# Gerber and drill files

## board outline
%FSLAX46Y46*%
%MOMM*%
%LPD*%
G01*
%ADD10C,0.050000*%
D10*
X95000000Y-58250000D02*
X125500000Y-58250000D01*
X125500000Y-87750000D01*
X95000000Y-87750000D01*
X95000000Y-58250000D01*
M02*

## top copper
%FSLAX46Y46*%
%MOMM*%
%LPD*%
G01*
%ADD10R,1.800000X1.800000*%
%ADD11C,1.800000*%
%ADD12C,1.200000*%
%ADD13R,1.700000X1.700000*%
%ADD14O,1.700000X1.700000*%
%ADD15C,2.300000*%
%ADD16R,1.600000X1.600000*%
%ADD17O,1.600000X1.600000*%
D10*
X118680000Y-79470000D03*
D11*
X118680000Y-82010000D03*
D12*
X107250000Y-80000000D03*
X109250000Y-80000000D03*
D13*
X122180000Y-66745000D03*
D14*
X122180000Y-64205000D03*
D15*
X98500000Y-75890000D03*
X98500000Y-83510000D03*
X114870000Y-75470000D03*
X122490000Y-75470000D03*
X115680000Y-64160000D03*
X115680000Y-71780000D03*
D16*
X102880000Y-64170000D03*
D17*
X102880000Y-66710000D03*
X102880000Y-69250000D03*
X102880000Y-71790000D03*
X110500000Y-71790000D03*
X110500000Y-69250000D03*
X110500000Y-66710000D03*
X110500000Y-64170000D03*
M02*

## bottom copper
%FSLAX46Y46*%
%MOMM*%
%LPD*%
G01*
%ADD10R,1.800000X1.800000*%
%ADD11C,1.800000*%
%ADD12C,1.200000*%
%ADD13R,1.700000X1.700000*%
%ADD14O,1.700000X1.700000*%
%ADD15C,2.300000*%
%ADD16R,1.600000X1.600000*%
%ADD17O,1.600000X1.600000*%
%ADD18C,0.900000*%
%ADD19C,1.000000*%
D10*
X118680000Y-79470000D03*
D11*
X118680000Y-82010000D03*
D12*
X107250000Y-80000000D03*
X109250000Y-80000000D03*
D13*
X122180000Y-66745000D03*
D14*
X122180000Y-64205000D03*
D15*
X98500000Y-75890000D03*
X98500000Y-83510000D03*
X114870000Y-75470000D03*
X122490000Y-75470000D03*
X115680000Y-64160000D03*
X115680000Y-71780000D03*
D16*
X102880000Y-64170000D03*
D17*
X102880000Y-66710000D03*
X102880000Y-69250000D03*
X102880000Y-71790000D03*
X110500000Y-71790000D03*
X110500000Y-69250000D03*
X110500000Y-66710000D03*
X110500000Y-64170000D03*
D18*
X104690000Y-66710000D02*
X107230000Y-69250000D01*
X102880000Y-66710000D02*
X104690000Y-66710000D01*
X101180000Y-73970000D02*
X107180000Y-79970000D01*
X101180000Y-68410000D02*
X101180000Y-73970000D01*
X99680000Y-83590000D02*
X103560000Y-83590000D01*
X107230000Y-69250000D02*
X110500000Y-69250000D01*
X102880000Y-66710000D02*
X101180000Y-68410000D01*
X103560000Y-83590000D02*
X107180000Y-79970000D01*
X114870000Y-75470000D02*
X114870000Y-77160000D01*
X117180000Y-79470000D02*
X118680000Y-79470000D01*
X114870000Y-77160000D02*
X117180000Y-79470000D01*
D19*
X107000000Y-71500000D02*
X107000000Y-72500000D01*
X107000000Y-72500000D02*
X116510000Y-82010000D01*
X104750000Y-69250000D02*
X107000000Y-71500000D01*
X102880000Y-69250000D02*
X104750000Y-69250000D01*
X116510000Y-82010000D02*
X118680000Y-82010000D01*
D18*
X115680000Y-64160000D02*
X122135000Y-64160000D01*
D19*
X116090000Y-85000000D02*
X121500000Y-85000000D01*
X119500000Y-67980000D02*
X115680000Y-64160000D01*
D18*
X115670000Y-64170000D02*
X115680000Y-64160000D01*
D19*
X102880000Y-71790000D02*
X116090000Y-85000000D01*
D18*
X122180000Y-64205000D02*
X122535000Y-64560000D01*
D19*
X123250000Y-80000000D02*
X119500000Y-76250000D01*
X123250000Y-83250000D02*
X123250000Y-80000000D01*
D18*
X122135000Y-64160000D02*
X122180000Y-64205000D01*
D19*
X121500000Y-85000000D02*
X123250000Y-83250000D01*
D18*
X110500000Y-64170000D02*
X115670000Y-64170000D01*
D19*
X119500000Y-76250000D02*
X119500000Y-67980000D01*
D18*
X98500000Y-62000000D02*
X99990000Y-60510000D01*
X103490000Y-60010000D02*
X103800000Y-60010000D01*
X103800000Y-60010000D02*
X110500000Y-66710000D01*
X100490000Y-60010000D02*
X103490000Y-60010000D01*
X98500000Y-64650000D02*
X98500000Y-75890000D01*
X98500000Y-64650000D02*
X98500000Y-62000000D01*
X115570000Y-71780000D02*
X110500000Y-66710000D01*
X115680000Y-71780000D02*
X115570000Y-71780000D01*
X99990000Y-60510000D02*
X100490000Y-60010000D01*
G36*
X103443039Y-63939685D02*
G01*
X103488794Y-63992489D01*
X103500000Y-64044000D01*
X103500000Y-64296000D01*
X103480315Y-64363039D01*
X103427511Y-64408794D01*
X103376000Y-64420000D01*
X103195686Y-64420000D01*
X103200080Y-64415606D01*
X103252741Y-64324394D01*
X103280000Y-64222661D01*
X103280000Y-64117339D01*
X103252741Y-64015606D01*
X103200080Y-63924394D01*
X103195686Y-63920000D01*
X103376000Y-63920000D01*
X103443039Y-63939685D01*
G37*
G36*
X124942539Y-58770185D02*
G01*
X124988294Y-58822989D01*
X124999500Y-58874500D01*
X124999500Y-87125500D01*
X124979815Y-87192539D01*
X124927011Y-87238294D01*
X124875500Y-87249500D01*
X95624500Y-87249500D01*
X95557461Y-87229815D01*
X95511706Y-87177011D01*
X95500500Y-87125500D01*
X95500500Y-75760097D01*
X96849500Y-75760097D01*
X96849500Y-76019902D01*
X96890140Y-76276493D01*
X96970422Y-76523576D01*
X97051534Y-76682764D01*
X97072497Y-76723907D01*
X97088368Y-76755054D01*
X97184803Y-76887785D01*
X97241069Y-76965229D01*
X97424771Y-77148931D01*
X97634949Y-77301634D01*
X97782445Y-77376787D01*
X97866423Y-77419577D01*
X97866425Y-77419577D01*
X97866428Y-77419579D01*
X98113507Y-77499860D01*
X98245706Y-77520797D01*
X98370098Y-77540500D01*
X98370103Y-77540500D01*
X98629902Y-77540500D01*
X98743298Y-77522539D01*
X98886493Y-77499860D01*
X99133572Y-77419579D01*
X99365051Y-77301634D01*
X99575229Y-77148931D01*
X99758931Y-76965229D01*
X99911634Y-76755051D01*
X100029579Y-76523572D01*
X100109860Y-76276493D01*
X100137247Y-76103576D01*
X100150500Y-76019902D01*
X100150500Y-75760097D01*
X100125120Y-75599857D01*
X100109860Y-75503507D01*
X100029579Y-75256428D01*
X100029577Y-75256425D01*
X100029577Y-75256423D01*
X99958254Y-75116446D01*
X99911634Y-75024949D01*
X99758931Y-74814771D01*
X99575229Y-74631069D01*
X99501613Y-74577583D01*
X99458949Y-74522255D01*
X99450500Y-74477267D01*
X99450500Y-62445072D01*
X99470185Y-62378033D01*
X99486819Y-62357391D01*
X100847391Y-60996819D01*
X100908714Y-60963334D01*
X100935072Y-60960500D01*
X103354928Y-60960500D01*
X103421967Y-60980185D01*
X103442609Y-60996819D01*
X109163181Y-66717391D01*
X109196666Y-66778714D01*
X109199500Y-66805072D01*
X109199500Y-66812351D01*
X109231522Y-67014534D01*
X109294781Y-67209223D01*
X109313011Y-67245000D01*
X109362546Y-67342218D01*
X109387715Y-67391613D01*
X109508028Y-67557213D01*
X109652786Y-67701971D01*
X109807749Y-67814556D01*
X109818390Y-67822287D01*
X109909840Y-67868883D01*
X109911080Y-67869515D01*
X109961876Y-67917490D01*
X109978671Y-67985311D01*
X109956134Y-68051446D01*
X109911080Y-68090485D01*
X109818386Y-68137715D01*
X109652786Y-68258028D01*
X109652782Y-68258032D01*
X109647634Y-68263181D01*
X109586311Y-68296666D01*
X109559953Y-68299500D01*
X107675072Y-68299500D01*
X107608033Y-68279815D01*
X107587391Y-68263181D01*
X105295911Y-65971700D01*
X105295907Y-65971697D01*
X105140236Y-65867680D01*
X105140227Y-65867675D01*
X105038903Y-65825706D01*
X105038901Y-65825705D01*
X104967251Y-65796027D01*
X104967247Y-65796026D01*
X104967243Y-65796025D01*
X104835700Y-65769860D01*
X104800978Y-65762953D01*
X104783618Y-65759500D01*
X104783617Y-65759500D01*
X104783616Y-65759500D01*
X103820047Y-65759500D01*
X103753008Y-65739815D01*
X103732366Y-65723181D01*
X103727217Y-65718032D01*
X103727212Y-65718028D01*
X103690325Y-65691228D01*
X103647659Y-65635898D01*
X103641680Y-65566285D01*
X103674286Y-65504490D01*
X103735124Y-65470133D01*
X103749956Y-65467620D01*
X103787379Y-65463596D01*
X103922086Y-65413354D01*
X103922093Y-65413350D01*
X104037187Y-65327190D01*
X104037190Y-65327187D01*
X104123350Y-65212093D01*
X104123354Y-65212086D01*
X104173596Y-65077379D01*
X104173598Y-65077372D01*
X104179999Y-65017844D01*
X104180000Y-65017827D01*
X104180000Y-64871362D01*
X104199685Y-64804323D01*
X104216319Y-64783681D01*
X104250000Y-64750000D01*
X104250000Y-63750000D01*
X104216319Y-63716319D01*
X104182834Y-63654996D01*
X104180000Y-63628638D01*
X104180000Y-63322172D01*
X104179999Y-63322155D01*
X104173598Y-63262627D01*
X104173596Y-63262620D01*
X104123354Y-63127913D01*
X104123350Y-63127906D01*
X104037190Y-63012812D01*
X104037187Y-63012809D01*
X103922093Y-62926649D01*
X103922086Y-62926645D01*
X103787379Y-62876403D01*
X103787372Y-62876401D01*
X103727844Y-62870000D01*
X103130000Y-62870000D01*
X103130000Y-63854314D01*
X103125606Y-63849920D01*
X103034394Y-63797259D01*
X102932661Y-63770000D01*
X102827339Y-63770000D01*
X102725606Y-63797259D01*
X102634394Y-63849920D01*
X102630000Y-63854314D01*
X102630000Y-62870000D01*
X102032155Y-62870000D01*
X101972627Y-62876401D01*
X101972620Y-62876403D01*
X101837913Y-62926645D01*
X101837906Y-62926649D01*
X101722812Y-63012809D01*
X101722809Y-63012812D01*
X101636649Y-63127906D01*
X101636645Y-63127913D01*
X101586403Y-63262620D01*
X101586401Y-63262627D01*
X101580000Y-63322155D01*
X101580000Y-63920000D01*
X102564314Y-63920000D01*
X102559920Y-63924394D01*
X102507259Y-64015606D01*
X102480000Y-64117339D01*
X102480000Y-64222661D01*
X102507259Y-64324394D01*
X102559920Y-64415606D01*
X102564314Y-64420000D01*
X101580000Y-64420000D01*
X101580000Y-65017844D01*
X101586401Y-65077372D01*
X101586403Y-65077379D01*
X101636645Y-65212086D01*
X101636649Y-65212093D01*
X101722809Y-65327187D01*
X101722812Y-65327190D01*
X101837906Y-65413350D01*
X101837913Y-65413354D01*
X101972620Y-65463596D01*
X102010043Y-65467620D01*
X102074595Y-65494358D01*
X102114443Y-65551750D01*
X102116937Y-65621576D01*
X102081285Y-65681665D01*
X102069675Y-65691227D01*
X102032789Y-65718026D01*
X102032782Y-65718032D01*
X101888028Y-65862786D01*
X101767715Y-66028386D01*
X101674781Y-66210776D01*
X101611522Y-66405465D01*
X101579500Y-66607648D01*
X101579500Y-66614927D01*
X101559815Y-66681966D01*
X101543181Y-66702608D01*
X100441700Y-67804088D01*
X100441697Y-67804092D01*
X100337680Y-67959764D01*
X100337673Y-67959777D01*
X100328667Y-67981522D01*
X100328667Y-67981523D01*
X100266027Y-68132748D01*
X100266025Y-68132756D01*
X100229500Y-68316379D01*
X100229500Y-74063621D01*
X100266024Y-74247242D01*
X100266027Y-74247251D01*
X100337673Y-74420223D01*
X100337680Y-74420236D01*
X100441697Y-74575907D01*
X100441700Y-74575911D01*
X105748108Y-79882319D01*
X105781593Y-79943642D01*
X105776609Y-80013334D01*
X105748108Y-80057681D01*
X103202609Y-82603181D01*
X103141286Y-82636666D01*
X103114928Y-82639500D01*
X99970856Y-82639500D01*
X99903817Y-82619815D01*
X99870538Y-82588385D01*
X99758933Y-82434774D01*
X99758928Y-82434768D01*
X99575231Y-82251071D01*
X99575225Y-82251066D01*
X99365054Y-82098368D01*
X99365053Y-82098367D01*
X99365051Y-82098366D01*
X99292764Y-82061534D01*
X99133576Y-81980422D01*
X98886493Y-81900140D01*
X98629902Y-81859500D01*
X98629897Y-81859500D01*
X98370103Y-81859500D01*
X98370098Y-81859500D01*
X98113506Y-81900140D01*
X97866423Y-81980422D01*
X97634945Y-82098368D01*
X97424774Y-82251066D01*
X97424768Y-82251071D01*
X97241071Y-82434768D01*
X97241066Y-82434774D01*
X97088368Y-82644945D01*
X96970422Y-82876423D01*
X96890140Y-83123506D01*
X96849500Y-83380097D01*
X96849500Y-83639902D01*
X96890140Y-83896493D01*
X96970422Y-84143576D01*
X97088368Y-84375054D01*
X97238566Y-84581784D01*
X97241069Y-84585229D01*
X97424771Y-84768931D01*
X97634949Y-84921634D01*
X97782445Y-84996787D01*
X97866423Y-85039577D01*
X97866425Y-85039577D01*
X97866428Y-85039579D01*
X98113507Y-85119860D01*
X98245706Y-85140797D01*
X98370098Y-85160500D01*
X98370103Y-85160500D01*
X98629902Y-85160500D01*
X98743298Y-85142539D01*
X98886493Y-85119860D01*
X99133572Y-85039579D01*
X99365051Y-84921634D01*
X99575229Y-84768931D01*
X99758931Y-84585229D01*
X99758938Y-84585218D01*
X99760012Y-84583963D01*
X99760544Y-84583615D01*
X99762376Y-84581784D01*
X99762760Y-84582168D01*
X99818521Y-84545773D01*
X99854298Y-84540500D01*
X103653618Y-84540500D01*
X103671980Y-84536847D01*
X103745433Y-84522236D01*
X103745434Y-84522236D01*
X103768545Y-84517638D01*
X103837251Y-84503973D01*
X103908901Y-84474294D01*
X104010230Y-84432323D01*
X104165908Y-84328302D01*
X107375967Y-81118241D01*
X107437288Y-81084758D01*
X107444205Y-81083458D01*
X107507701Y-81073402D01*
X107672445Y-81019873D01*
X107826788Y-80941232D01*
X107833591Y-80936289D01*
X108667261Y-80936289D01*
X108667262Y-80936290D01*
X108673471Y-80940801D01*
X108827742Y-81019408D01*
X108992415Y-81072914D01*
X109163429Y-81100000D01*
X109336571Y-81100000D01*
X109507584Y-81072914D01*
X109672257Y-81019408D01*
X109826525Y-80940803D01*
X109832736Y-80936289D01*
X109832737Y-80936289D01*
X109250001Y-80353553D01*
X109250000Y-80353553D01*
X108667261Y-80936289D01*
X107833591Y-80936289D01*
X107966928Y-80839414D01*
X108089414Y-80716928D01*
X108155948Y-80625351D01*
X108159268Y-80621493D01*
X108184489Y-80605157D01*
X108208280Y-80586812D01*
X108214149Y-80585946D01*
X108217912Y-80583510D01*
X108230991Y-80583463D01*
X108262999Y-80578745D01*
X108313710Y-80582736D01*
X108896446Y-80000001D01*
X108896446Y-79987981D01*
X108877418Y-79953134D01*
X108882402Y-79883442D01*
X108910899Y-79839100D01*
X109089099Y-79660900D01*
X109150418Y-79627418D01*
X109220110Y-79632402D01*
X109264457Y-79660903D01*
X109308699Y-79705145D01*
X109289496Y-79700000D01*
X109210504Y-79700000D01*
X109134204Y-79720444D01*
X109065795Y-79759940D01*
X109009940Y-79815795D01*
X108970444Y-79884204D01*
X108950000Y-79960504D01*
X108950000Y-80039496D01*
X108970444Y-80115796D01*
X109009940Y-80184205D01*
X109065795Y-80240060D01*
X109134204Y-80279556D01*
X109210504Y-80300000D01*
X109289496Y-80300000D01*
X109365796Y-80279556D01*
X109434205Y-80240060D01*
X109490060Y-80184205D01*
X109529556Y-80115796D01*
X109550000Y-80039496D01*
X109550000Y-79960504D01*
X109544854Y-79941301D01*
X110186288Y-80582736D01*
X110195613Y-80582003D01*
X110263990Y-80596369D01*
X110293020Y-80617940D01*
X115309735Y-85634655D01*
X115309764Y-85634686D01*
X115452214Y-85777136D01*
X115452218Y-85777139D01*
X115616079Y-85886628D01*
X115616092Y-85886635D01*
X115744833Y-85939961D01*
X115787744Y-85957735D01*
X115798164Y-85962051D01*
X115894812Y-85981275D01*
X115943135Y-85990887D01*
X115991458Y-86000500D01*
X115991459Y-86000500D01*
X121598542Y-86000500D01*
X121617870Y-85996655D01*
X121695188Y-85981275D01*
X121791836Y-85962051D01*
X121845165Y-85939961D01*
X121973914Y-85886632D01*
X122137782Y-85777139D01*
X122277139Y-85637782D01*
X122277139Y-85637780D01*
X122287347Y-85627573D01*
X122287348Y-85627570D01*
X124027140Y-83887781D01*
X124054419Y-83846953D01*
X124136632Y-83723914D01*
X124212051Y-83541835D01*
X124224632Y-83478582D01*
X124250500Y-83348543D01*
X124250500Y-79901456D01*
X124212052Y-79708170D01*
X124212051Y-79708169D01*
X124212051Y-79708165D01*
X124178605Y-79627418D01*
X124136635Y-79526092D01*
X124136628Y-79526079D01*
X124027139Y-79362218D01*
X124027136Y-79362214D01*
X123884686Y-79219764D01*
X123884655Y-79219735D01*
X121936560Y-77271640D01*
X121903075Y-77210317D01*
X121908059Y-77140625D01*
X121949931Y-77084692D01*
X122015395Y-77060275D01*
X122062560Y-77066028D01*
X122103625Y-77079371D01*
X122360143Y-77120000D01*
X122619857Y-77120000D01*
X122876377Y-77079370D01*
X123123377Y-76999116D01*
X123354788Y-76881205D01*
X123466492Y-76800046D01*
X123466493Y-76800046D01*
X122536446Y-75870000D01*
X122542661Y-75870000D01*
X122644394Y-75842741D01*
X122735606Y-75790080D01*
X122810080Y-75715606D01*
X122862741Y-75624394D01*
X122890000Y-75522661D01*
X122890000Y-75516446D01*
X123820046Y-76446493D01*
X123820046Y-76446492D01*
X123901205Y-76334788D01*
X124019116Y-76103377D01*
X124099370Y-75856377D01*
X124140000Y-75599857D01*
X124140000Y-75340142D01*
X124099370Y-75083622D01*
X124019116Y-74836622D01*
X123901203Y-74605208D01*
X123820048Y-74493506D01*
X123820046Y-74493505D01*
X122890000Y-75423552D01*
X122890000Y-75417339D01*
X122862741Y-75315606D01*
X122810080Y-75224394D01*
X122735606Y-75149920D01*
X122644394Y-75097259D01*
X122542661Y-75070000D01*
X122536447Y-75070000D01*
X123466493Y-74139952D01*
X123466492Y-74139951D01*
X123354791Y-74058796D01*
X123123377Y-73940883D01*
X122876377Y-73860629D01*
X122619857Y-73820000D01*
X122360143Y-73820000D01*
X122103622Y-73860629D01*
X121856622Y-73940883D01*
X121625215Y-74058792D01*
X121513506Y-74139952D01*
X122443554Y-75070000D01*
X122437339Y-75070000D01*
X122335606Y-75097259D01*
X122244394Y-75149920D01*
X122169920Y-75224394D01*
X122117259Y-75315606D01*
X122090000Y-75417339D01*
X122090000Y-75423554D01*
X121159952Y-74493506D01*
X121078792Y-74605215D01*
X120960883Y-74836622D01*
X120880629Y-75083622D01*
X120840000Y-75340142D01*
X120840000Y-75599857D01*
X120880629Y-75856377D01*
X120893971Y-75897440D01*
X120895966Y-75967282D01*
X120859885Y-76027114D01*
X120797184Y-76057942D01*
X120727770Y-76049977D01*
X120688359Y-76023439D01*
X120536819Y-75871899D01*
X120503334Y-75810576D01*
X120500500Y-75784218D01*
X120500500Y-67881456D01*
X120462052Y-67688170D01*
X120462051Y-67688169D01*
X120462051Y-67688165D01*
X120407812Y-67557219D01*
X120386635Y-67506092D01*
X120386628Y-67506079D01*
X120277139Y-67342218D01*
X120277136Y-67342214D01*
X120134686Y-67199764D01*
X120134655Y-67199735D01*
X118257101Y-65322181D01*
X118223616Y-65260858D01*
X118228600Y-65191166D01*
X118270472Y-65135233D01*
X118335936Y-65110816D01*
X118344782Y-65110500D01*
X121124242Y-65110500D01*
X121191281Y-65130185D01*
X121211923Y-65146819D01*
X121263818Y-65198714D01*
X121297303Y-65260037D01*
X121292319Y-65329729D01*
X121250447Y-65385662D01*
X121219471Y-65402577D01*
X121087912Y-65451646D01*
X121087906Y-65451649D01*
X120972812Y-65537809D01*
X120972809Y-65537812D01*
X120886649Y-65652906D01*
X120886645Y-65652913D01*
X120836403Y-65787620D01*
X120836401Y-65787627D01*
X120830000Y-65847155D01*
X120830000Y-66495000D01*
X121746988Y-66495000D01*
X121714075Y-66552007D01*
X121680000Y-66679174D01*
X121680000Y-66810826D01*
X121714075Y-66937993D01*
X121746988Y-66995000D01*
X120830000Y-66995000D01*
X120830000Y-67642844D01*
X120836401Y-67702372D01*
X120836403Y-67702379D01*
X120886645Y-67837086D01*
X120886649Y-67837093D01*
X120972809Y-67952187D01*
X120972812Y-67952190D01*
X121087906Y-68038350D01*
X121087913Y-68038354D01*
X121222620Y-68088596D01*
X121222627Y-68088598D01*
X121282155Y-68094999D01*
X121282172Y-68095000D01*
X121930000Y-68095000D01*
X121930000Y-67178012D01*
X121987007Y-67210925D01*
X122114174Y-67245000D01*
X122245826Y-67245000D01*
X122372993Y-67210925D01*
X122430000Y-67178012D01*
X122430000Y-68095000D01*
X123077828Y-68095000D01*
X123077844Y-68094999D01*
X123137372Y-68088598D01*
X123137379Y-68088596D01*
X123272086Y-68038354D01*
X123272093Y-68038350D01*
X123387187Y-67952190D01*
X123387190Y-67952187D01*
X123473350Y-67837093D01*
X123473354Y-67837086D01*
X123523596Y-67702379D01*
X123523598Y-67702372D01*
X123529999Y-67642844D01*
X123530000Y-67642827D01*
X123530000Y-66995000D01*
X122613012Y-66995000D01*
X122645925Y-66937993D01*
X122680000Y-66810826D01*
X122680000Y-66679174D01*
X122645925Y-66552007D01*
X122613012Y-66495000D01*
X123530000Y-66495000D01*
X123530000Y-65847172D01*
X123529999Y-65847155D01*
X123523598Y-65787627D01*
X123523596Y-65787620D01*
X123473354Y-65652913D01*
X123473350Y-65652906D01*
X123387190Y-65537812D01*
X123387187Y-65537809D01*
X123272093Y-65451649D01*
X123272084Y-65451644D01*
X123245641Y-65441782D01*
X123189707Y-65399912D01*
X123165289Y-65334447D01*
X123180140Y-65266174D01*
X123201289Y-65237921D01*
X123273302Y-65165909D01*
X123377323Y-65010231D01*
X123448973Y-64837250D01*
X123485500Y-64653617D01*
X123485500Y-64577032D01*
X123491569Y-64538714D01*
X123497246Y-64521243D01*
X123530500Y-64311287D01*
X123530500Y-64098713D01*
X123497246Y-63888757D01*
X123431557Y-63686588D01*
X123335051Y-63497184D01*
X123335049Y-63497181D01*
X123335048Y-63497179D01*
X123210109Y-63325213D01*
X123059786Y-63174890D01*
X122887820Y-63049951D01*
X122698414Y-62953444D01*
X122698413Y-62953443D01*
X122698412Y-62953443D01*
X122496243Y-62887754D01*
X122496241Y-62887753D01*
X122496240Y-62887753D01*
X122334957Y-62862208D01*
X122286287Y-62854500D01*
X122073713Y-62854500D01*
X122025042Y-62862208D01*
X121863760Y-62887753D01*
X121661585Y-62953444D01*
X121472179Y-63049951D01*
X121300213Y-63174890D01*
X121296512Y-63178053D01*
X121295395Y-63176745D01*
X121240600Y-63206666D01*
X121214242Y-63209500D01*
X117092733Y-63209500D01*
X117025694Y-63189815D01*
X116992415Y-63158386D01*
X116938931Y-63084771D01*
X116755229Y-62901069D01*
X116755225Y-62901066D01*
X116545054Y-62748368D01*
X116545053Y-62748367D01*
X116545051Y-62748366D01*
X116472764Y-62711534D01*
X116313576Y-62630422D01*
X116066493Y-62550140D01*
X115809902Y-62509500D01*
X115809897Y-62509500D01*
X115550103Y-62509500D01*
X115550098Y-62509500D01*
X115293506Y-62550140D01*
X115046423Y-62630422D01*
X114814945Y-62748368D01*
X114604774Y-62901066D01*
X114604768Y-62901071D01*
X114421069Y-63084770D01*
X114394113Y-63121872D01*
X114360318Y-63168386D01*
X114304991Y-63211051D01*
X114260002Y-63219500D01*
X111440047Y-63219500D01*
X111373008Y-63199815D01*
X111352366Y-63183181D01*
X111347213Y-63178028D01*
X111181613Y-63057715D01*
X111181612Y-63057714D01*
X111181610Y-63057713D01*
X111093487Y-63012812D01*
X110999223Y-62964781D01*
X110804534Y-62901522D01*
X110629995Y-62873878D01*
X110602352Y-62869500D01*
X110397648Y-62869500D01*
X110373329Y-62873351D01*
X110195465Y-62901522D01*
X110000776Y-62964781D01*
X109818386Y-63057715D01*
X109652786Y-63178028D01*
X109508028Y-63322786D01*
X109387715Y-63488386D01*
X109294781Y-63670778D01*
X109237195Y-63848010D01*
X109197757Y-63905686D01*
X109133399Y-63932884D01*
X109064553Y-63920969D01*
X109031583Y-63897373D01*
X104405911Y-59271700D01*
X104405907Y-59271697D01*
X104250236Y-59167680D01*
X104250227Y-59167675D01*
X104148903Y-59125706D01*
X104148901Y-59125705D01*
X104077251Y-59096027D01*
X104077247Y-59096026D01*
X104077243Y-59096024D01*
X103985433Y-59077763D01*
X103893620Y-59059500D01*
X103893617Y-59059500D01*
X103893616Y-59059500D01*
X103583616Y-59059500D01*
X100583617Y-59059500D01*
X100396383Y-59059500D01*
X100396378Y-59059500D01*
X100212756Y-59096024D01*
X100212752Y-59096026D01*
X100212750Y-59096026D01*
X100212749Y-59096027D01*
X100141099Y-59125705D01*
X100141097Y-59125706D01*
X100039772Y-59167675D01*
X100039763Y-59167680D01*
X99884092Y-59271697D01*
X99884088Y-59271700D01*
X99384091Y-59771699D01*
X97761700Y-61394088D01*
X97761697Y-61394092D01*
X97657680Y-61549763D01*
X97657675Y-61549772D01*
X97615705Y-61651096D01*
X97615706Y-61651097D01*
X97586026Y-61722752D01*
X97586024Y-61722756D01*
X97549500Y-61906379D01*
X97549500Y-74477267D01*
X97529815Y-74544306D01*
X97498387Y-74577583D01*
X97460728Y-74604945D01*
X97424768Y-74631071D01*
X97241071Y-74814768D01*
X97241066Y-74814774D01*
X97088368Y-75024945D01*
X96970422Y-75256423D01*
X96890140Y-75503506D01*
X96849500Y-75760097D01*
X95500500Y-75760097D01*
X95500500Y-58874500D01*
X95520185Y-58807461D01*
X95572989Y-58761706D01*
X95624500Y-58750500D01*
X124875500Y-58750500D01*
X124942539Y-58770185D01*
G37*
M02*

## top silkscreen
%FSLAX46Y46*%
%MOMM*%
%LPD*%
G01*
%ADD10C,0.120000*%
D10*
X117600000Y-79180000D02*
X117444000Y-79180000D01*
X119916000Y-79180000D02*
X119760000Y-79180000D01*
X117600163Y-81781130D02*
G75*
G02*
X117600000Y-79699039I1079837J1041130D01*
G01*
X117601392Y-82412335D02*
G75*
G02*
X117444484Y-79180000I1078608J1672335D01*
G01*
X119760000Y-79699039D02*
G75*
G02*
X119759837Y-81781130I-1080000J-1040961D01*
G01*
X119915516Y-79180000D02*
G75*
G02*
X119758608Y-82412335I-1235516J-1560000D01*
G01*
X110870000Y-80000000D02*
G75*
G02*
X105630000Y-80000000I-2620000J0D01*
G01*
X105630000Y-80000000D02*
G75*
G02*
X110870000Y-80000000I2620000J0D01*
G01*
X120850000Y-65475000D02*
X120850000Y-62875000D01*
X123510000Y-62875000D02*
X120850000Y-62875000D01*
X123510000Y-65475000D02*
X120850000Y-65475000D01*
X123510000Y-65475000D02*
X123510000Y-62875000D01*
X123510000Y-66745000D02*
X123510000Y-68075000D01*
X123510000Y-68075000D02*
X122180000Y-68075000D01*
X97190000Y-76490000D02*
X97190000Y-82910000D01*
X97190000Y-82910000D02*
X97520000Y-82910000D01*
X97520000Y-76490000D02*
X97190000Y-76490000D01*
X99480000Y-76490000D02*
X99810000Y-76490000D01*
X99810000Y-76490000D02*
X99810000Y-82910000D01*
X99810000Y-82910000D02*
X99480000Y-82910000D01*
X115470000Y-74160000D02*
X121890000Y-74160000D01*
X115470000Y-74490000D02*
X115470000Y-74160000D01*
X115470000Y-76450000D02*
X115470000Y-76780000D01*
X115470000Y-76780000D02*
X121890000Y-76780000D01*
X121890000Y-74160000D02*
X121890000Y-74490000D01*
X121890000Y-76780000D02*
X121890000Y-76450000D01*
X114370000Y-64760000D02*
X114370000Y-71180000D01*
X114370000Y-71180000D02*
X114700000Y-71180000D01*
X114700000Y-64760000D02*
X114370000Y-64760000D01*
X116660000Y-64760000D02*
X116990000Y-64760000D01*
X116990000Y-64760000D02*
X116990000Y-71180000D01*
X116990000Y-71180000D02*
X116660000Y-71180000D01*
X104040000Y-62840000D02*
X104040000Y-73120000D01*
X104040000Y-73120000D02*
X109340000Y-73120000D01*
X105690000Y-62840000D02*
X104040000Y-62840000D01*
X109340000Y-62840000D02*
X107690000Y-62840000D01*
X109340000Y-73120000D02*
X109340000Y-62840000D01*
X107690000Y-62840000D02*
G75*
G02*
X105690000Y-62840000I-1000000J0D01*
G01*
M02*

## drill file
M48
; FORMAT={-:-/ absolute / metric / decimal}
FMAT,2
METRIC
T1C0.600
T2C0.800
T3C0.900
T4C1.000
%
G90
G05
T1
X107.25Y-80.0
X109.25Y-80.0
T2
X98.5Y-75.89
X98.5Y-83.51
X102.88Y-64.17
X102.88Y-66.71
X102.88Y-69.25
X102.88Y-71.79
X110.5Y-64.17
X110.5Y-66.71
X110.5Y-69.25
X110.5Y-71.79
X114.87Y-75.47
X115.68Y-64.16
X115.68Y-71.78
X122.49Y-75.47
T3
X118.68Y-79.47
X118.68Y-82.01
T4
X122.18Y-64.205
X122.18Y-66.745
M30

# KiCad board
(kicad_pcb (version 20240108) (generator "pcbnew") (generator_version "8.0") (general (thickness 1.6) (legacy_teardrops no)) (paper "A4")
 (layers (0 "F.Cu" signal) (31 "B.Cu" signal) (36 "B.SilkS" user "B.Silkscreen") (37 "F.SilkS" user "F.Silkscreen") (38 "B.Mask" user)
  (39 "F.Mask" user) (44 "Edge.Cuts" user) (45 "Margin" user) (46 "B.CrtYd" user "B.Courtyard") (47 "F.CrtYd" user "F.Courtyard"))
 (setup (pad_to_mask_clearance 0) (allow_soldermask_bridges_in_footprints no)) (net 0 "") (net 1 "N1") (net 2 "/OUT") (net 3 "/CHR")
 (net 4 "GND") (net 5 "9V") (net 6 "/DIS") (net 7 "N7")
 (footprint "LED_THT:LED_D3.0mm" (layer "F.Cu") (at 118.68 79.47 -90)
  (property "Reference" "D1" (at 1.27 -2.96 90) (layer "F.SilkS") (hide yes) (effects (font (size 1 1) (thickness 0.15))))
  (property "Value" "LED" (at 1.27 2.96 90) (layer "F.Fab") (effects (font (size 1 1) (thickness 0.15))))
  (fp_line (start -0.29 1.08) (end -0.29 1.236) (stroke (width 0.12) (type solid)) (layer "F.SilkS"))
  (fp_line (start -0.29 -1.236) (end -0.29 -1.08) (stroke (width 0.12) (type solid)) (layer "F.SilkS"))
  (fp_arc (start 2.31113 1.079837) (mid 1.270117 1.5) (end 0.229039 1.08) (stroke (width 0.12) (type solid)) (layer "F.SilkS"))
  (fp_arc (start 2.942335 1.078608) (mid 1.366487 1.987659) (end -0.29 1.235516) (stroke (width 0.12) (type solid)) (layer "F.SilkS"))
  (fp_arc (start 0.229039 -1.08) (mid 1.270117 -1.5) (end 2.31113 -1.079837) (stroke (width 0.12) (type solid)) (layer "F.SilkS"))
  (fp_arc (start -0.29 -1.235516) (mid 1.366487 -1.987659) (end 2.942335 -1.078608) (stroke (width 0.12) (type solid)) (layer "F.SilkS"))
  (pad "1" thru_hole rect (at 0 0 270) (size 1.8 1.8) (drill 0.9) (layers "*.Cu" "*.Mask") (remove_unused_layers no) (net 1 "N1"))
  (pad "2" thru_hole circle (at 2.54 0 270) (size 1.8 1.8) (drill 0.9) (layers "*.Cu" "*.Mask") (remove_unused_layers no) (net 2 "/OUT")))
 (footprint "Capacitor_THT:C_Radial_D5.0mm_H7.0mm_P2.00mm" (layer "F.Cu") (at 107.25 80)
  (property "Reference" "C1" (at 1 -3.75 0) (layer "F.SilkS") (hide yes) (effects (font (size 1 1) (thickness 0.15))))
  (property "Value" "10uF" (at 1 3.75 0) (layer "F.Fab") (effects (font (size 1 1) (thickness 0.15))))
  (fp_circle (center 1 0) (end 3.62 0) (stroke (width 0.12) (type solid)) (fill none) (layer "F.SilkS"))
  (pad "1" thru_hole circle (at 0 0) (size 1.2 1.2) (drill 0.6) (layers "*.Cu" "*.Mask") (remove_unused_layers no) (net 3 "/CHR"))
  (pad "2" thru_hole circle (at 2 0) (size 1.2 1.2) (drill 0.6) (layers "*.Cu" "*.Mask") (remove_unused_layers no) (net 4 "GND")))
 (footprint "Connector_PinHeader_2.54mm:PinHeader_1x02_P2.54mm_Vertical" (layer "F.Cu") (at 122.18 66.745 180)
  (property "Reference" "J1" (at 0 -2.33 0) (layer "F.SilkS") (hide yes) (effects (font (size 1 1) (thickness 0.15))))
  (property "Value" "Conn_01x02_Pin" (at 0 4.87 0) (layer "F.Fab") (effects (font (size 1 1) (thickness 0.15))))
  (fp_line (start 1.33 1.27) (end 1.33 3.87) (stroke (width 0.12) (type solid)) (layer "F.SilkS"))
  (fp_line (start -1.33 3.87) (end 1.33 3.87) (stroke (width 0.12) (type solid)) (layer "F.SilkS"))
  (fp_line (start -1.33 1.27) (end 1.33 1.27) (stroke (width 0.12) (type solid)) (layer "F.SilkS"))
  (fp_line (start -1.33 1.27) (end -1.33 3.87) (stroke (width 0.12) (type solid)) (layer "F.SilkS"))
  (fp_line (start -1.33 0) (end -1.33 -1.33) (stroke (width 0.12) (type solid)) (layer "F.SilkS"))
  (fp_line (start -1.33 -1.33) (end 0 -1.33) (stroke (width 0.12) (type solid)) (layer "F.SilkS"))
  (pad "1" thru_hole rect (at 0 0 180) (size 1.7 1.7) (drill 1) (layers "*.Cu" "*.Mask") (remove_unused_layers no) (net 4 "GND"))
  (pad "2" thru_hole oval (at 0 2.54 180) (size 1.7 1.7) (drill 1) (layers "*.Cu" "*.Mask") (remove_unused_layers no) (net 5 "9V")))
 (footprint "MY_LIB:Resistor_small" (layer "F.Cu") (at 98.5 75.89 -90)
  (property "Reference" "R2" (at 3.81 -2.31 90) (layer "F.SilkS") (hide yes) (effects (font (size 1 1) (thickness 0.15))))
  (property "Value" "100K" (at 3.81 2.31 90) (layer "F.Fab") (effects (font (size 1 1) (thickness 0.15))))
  (fp_line (start 0.6 1.31) (end 7.02 1.31) (stroke (width 0.12) (type solid)) (layer "F.SilkS"))
  (fp_line (start 7.02 1.31) (end 7.02 0.98) (stroke (width 0.12) (type solid)) (layer "F.SilkS"))
  (fp_line (start 0.6 0.98) (end 0.6 1.31) (stroke (width 0.12) (type solid)) (layer "F.SilkS"))
  (fp_line (start 0.6 -0.98) (end 0.6 -1.31) (stroke (width 0.12) (type solid)) (layer "F.SilkS"))
  (fp_line (start 0.6 -1.31) (end 7.02 -1.31) (stroke (width 0.12) (type solid)) (layer "F.SilkS"))
  (fp_line (start 7.02 -1.31) (end 7.02 -0.98) (stroke (width 0.12) (type solid)) (layer "F.SilkS"))
  (pad "1" thru_hole circle (at 0 0 270) (size 2.3 2.3) (drill 0.8) (layers "*.Cu" "*.Mask") (remove_unused_layers no) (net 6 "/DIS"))
  (pad "2" thru_hole circle (at 7.62 0 270) (size 2.3 2.3) (drill 0.8) (layers "*.Cu" "*.Mask") (remove_unused_layers no) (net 3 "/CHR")))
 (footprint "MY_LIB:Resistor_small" (layer "F.Cu") (at 114.87 75.47)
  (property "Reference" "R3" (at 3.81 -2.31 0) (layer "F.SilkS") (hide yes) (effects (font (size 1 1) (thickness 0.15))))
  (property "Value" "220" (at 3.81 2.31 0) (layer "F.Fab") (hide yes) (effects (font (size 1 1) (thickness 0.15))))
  (fp_line (start 0.6 -1.31) (end 7.02 -1.31) (stroke (width 0.12) (type solid)) (layer "F.SilkS"))
  (fp_line (start 0.6 -0.98) (end 0.6 -1.31) (stroke (width 0.12) (type solid)) (layer "F.SilkS"))
  (fp_line (start 0.6 0.98) (end 0.6 1.31) (stroke (width 0.12) (type solid)) (layer "F.SilkS"))
  (fp_line (start 0.6 1.31) (end 7.02 1.31) (stroke (width 0.12) (type solid)) (layer "F.SilkS"))
  (fp_line (start 7.02 -1.31) (end 7.02 -0.98) (stroke (width 0.12) (type solid)) (layer "F.SilkS"))
  (fp_line (start 7.02 1.31) (end 7.02 0.98) (stroke (width 0.12) (type solid)) (layer "F.SilkS"))
  (pad "1" thru_hole circle (at 0 0) (size 2.3 2.3) (drill 0.8) (layers "*.Cu" "*.Mask") (remove_unused_layers no) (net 1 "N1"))
  (pad "2" thru_hole circle (at 7.62 0) (size 2.3 2.3) (drill 0.8) (layers "*.Cu" "*.Mask") (remove_unused_layers no) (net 4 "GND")))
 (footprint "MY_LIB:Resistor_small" (layer "F.Cu") (at 115.68 64.16 -90)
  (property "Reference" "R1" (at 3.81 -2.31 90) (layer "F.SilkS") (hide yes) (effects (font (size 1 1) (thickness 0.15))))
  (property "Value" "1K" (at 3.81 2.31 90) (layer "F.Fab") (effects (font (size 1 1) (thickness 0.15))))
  (fp_line (start 0.6 1.31) (end 7.02 1.31) (stroke (width 0.12) (type solid)) (layer "F.SilkS"))
  (fp_line (start 7.02 1.31) (end 7.02 0.98) (stroke (width 0.12) (type solid)) (layer "F.SilkS"))
  (fp_line (start 0.6 0.98) (end 0.6 1.31) (stroke (width 0.12) (type solid)) (layer "F.SilkS"))
  (fp_line (start 0.6 -0.98) (end 0.6 -1.31) (stroke (width 0.12) (type solid)) (layer "F.SilkS"))
  (fp_line (start 0.6 -1.31) (end 7.02 -1.31) (stroke (width 0.12) (type solid)) (layer "F.SilkS"))
  (fp_line (start 7.02 -1.31) (end 7.02 -0.98) (stroke (width 0.12) (type solid)) (layer "F.SilkS"))
  (pad "1" thru_hole circle (at 0 0 270) (size 2.3 2.3) (drill 0.8) (layers "*.Cu" "*.Mask") (remove_unused_layers no) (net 5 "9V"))
  (pad "2" thru_hole circle (at 7.62 0 270) (size 2.3 2.3) (drill 0.8) (layers "*.Cu" "*.Mask") (remove_unused_layers no) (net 6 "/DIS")))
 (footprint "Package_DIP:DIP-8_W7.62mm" (layer "F.Cu") (at 102.88 64.17)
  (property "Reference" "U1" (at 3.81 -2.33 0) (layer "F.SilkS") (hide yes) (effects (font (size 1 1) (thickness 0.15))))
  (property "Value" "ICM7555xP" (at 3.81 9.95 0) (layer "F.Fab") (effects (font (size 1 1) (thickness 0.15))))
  (fp_line (start 1.16 -1.33) (end 1.16 8.95) (stroke (width 0.12) (type solid)) (layer "F.SilkS"))
  (fp_line (start 1.16 8.95) (end 6.46 8.95) (stroke (width 0.12) (type solid)) (layer "F.SilkS"))
  (fp_line (start 2.81 -1.33) (end 1.16 -1.33) (stroke (width 0.12) (type solid)) (layer "F.SilkS"))
  (fp_line (start 6.46 -1.33) (end 4.81 -1.33) (stroke (width 0.12) (type solid)) (layer "F.SilkS"))
  (fp_line (start 6.46 8.95) (end 6.46 -1.33) (stroke (width 0.12) (type solid)) (layer "F.SilkS"))
  (fp_arc (start 4.81 -1.33) (mid 3.81 -0.33) (end 2.81 -1.33) (stroke (width 0.12) (type solid)) (layer "F.SilkS"))
  (pad "1" thru_hole rect (at 0 0) (size 1.6 1.6) (drill 0.8) (layers "*.Cu" "*.Mask") (remove_unused_layers no) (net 4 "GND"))
  (pad "2" thru_hole oval (at 0 2.54) (size 1.6 1.6) (drill 0.8) (layers "*.Cu" "*.Mask") (remove_unused_layers no) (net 3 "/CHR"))
  (pad "3" thru_hole oval (at 0 5.08) (size 1.6 1.6) (drill 0.8) (layers "*.Cu" "*.Mask") (remove_unused_layers no) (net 2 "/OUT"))
  (pad "4" thru_hole oval (at 0 7.62) (size 1.6 1.6) (drill 0.8) (layers "*.Cu" "*.Mask") (remove_unused_layers no) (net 5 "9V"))
  (pad "5" thru_hole oval (at 7.62 7.62) (size 1.6 1.6) (drill 0.8) (layers "*.Cu" "*.Mask") (remove_unused_layers no) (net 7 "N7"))
  (pad "6" thru_hole oval (at 7.62 5.08) (size 1.6 1.6) (drill 0.8) (layers "*.Cu" "*.Mask") (remove_unused_layers no) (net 3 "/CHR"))
  (pad "7" thru_hole oval (at 7.62 2.54) (size 1.6 1.6) (drill 0.8) (layers "*.Cu" "*.Mask") (remove_unused_layers no) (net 6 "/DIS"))
  (pad "8" thru_hole oval (at 7.62 0) (size 1.6 1.6) (drill 0.8) (layers "*.Cu" "*.Mask") (remove_unused_layers no) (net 5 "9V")))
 (gr_rect (start 95 58.25) (end 125.5 87.75) (stroke (width 0.05) (type default)) (fill none) (layer "Edge.Cuts"))
 (segment (start 104.69 66.71) (end 107.23 69.25) (width 0.9) (layer "B.Cu") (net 3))
 (segment (start 102.88 66.71) (end 104.69 66.71) (width 0.9) (layer "B.Cu") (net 3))
 (segment (start 101.18 73.97) (end 107.18 79.97) (width 0.9) (layer "B.Cu") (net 3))
 (segment (start 101.18 68.41) (end 101.18 73.97) (width 0.9) (layer "B.Cu") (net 3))
 (segment (start 99.68 83.59) (end 103.56 83.59) (width 0.9) (layer "B.Cu") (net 3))
 (segment (start 107.23 69.25) (end 110.5 69.25) (width 0.9) (layer "B.Cu") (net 3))
 (segment (start 102.88 66.71) (end 101.18 68.41) (width 0.9) (layer "B.Cu") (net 3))
 (segment (start 103.56 83.59) (end 107.18 79.97) (width 0.9) (layer "B.Cu") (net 3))
 (segment (start 114.87 75.47) (end 114.87 77.16) (width 0.9) (layer "B.Cu") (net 1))
 (segment (start 117.18 79.47) (end 118.68 79.47) (width 0.9) (layer "B.Cu") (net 1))
 (segment (start 114.87 77.16) (end 117.18 79.47) (width 0.9) (layer "B.Cu") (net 1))
 (segment (start 107 71.5) (end 107 72.5) (width 1) (layer "B.Cu") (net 2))
 (segment (start 107 72.5) (end 116.51 82.01) (width 1) (layer "B.Cu") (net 2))
 (segment (start 104.75 69.25) (end 107 71.5) (width 1) (layer "B.Cu") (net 2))
 (segment (start 102.88 69.25) (end 104.75 69.25) (width 1) (layer "B.Cu") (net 2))
 (segment (start 116.51 82.01) (end 118.68 82.01) (width 1) (layer "B.Cu") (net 2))
 (segment (start 115.68 64.16) (end 122.135 64.16) (width 0.9) (layer "B.Cu") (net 5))
 (segment (start 116.09 85) (end 121.5 85) (width 1) (layer "B.Cu") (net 5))
 (segment (start 119.5 67.98) (end 115.68 64.16) (width 1) (layer "B.Cu") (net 5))
 (segment (start 115.67 64.17) (end 115.68 64.16) (width 0.9) (layer "B.Cu") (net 5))
 (segment (start 102.88 71.79) (end 116.09 85) (width 1) (layer "B.Cu") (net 5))
 (segment (start 122.18 64.205) (end 122.535 64.56) (width 0.9) (layer "B.Cu") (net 5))
 (segment (start 123.25 80) (end 119.5 76.25) (width 1) (layer "B.Cu") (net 5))
 (segment (start 123.25 83.25) (end 123.25 80) (width 1) (layer "B.Cu") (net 5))
 (segment (start 122.135 64.16) (end 122.18 64.205) (width 0.9) (layer "B.Cu") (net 5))
 (segment (start 121.5 85) (end 123.25 83.25) (width 1) (layer "B.Cu") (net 5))
 (segment (start 110.5 64.17) (end 115.67 64.17) (width 0.9) (layer "B.Cu") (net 5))
 (segment (start 119.5 76.25) (end 119.5 67.98) (width 1) (layer "B.Cu") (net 5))
 (segment (start 98.5 62) (end 99.99 60.51) (width 0.9) (layer "B.Cu") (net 6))
 (segment (start 103.49 60.01) (end 103.8 60.01) (width 0.9) (layer "B.Cu") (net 6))
 (segment (start 103.8 60.01) (end 110.5 66.71) (width 0.9) (layer "B.Cu") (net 6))
 (segment (start 100.49 60.01) (end 103.49 60.01) (width 0.9) (layer "B.Cu") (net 6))
 (segment (start 98.5 64.65) (end 98.5 75.89) (width 0.9) (layer "B.Cu") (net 6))
 (segment (start 98.5 64.65) (end 98.5 62) (width 0.9) (layer "B.Cu") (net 6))
 (segment (start 115.57 71.78) (end 110.5 66.71) (width 0.9) (layer "B.Cu") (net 6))
 (segment (start 115.68 71.78) (end 115.57 71.78) (width 0.9) (layer "B.Cu") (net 6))
 (segment (start 99.99 60.51) (end 100.49 60.01) (width 0.9) (layer "B.Cu") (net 6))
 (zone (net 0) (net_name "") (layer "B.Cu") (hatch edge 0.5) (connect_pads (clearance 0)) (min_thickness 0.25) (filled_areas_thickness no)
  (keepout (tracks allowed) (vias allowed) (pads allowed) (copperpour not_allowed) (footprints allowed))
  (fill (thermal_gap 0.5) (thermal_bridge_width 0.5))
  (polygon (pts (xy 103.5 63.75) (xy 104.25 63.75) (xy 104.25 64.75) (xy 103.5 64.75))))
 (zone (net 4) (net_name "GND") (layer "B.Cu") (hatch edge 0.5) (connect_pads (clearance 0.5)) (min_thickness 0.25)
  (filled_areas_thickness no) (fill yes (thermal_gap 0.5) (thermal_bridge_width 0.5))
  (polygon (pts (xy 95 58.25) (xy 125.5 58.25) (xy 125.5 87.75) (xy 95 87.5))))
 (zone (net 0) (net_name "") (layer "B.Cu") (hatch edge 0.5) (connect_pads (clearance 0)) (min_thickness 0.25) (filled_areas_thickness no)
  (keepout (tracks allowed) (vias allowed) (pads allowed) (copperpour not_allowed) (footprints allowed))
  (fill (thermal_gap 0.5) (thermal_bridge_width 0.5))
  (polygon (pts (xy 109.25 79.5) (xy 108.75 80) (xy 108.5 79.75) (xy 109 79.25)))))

